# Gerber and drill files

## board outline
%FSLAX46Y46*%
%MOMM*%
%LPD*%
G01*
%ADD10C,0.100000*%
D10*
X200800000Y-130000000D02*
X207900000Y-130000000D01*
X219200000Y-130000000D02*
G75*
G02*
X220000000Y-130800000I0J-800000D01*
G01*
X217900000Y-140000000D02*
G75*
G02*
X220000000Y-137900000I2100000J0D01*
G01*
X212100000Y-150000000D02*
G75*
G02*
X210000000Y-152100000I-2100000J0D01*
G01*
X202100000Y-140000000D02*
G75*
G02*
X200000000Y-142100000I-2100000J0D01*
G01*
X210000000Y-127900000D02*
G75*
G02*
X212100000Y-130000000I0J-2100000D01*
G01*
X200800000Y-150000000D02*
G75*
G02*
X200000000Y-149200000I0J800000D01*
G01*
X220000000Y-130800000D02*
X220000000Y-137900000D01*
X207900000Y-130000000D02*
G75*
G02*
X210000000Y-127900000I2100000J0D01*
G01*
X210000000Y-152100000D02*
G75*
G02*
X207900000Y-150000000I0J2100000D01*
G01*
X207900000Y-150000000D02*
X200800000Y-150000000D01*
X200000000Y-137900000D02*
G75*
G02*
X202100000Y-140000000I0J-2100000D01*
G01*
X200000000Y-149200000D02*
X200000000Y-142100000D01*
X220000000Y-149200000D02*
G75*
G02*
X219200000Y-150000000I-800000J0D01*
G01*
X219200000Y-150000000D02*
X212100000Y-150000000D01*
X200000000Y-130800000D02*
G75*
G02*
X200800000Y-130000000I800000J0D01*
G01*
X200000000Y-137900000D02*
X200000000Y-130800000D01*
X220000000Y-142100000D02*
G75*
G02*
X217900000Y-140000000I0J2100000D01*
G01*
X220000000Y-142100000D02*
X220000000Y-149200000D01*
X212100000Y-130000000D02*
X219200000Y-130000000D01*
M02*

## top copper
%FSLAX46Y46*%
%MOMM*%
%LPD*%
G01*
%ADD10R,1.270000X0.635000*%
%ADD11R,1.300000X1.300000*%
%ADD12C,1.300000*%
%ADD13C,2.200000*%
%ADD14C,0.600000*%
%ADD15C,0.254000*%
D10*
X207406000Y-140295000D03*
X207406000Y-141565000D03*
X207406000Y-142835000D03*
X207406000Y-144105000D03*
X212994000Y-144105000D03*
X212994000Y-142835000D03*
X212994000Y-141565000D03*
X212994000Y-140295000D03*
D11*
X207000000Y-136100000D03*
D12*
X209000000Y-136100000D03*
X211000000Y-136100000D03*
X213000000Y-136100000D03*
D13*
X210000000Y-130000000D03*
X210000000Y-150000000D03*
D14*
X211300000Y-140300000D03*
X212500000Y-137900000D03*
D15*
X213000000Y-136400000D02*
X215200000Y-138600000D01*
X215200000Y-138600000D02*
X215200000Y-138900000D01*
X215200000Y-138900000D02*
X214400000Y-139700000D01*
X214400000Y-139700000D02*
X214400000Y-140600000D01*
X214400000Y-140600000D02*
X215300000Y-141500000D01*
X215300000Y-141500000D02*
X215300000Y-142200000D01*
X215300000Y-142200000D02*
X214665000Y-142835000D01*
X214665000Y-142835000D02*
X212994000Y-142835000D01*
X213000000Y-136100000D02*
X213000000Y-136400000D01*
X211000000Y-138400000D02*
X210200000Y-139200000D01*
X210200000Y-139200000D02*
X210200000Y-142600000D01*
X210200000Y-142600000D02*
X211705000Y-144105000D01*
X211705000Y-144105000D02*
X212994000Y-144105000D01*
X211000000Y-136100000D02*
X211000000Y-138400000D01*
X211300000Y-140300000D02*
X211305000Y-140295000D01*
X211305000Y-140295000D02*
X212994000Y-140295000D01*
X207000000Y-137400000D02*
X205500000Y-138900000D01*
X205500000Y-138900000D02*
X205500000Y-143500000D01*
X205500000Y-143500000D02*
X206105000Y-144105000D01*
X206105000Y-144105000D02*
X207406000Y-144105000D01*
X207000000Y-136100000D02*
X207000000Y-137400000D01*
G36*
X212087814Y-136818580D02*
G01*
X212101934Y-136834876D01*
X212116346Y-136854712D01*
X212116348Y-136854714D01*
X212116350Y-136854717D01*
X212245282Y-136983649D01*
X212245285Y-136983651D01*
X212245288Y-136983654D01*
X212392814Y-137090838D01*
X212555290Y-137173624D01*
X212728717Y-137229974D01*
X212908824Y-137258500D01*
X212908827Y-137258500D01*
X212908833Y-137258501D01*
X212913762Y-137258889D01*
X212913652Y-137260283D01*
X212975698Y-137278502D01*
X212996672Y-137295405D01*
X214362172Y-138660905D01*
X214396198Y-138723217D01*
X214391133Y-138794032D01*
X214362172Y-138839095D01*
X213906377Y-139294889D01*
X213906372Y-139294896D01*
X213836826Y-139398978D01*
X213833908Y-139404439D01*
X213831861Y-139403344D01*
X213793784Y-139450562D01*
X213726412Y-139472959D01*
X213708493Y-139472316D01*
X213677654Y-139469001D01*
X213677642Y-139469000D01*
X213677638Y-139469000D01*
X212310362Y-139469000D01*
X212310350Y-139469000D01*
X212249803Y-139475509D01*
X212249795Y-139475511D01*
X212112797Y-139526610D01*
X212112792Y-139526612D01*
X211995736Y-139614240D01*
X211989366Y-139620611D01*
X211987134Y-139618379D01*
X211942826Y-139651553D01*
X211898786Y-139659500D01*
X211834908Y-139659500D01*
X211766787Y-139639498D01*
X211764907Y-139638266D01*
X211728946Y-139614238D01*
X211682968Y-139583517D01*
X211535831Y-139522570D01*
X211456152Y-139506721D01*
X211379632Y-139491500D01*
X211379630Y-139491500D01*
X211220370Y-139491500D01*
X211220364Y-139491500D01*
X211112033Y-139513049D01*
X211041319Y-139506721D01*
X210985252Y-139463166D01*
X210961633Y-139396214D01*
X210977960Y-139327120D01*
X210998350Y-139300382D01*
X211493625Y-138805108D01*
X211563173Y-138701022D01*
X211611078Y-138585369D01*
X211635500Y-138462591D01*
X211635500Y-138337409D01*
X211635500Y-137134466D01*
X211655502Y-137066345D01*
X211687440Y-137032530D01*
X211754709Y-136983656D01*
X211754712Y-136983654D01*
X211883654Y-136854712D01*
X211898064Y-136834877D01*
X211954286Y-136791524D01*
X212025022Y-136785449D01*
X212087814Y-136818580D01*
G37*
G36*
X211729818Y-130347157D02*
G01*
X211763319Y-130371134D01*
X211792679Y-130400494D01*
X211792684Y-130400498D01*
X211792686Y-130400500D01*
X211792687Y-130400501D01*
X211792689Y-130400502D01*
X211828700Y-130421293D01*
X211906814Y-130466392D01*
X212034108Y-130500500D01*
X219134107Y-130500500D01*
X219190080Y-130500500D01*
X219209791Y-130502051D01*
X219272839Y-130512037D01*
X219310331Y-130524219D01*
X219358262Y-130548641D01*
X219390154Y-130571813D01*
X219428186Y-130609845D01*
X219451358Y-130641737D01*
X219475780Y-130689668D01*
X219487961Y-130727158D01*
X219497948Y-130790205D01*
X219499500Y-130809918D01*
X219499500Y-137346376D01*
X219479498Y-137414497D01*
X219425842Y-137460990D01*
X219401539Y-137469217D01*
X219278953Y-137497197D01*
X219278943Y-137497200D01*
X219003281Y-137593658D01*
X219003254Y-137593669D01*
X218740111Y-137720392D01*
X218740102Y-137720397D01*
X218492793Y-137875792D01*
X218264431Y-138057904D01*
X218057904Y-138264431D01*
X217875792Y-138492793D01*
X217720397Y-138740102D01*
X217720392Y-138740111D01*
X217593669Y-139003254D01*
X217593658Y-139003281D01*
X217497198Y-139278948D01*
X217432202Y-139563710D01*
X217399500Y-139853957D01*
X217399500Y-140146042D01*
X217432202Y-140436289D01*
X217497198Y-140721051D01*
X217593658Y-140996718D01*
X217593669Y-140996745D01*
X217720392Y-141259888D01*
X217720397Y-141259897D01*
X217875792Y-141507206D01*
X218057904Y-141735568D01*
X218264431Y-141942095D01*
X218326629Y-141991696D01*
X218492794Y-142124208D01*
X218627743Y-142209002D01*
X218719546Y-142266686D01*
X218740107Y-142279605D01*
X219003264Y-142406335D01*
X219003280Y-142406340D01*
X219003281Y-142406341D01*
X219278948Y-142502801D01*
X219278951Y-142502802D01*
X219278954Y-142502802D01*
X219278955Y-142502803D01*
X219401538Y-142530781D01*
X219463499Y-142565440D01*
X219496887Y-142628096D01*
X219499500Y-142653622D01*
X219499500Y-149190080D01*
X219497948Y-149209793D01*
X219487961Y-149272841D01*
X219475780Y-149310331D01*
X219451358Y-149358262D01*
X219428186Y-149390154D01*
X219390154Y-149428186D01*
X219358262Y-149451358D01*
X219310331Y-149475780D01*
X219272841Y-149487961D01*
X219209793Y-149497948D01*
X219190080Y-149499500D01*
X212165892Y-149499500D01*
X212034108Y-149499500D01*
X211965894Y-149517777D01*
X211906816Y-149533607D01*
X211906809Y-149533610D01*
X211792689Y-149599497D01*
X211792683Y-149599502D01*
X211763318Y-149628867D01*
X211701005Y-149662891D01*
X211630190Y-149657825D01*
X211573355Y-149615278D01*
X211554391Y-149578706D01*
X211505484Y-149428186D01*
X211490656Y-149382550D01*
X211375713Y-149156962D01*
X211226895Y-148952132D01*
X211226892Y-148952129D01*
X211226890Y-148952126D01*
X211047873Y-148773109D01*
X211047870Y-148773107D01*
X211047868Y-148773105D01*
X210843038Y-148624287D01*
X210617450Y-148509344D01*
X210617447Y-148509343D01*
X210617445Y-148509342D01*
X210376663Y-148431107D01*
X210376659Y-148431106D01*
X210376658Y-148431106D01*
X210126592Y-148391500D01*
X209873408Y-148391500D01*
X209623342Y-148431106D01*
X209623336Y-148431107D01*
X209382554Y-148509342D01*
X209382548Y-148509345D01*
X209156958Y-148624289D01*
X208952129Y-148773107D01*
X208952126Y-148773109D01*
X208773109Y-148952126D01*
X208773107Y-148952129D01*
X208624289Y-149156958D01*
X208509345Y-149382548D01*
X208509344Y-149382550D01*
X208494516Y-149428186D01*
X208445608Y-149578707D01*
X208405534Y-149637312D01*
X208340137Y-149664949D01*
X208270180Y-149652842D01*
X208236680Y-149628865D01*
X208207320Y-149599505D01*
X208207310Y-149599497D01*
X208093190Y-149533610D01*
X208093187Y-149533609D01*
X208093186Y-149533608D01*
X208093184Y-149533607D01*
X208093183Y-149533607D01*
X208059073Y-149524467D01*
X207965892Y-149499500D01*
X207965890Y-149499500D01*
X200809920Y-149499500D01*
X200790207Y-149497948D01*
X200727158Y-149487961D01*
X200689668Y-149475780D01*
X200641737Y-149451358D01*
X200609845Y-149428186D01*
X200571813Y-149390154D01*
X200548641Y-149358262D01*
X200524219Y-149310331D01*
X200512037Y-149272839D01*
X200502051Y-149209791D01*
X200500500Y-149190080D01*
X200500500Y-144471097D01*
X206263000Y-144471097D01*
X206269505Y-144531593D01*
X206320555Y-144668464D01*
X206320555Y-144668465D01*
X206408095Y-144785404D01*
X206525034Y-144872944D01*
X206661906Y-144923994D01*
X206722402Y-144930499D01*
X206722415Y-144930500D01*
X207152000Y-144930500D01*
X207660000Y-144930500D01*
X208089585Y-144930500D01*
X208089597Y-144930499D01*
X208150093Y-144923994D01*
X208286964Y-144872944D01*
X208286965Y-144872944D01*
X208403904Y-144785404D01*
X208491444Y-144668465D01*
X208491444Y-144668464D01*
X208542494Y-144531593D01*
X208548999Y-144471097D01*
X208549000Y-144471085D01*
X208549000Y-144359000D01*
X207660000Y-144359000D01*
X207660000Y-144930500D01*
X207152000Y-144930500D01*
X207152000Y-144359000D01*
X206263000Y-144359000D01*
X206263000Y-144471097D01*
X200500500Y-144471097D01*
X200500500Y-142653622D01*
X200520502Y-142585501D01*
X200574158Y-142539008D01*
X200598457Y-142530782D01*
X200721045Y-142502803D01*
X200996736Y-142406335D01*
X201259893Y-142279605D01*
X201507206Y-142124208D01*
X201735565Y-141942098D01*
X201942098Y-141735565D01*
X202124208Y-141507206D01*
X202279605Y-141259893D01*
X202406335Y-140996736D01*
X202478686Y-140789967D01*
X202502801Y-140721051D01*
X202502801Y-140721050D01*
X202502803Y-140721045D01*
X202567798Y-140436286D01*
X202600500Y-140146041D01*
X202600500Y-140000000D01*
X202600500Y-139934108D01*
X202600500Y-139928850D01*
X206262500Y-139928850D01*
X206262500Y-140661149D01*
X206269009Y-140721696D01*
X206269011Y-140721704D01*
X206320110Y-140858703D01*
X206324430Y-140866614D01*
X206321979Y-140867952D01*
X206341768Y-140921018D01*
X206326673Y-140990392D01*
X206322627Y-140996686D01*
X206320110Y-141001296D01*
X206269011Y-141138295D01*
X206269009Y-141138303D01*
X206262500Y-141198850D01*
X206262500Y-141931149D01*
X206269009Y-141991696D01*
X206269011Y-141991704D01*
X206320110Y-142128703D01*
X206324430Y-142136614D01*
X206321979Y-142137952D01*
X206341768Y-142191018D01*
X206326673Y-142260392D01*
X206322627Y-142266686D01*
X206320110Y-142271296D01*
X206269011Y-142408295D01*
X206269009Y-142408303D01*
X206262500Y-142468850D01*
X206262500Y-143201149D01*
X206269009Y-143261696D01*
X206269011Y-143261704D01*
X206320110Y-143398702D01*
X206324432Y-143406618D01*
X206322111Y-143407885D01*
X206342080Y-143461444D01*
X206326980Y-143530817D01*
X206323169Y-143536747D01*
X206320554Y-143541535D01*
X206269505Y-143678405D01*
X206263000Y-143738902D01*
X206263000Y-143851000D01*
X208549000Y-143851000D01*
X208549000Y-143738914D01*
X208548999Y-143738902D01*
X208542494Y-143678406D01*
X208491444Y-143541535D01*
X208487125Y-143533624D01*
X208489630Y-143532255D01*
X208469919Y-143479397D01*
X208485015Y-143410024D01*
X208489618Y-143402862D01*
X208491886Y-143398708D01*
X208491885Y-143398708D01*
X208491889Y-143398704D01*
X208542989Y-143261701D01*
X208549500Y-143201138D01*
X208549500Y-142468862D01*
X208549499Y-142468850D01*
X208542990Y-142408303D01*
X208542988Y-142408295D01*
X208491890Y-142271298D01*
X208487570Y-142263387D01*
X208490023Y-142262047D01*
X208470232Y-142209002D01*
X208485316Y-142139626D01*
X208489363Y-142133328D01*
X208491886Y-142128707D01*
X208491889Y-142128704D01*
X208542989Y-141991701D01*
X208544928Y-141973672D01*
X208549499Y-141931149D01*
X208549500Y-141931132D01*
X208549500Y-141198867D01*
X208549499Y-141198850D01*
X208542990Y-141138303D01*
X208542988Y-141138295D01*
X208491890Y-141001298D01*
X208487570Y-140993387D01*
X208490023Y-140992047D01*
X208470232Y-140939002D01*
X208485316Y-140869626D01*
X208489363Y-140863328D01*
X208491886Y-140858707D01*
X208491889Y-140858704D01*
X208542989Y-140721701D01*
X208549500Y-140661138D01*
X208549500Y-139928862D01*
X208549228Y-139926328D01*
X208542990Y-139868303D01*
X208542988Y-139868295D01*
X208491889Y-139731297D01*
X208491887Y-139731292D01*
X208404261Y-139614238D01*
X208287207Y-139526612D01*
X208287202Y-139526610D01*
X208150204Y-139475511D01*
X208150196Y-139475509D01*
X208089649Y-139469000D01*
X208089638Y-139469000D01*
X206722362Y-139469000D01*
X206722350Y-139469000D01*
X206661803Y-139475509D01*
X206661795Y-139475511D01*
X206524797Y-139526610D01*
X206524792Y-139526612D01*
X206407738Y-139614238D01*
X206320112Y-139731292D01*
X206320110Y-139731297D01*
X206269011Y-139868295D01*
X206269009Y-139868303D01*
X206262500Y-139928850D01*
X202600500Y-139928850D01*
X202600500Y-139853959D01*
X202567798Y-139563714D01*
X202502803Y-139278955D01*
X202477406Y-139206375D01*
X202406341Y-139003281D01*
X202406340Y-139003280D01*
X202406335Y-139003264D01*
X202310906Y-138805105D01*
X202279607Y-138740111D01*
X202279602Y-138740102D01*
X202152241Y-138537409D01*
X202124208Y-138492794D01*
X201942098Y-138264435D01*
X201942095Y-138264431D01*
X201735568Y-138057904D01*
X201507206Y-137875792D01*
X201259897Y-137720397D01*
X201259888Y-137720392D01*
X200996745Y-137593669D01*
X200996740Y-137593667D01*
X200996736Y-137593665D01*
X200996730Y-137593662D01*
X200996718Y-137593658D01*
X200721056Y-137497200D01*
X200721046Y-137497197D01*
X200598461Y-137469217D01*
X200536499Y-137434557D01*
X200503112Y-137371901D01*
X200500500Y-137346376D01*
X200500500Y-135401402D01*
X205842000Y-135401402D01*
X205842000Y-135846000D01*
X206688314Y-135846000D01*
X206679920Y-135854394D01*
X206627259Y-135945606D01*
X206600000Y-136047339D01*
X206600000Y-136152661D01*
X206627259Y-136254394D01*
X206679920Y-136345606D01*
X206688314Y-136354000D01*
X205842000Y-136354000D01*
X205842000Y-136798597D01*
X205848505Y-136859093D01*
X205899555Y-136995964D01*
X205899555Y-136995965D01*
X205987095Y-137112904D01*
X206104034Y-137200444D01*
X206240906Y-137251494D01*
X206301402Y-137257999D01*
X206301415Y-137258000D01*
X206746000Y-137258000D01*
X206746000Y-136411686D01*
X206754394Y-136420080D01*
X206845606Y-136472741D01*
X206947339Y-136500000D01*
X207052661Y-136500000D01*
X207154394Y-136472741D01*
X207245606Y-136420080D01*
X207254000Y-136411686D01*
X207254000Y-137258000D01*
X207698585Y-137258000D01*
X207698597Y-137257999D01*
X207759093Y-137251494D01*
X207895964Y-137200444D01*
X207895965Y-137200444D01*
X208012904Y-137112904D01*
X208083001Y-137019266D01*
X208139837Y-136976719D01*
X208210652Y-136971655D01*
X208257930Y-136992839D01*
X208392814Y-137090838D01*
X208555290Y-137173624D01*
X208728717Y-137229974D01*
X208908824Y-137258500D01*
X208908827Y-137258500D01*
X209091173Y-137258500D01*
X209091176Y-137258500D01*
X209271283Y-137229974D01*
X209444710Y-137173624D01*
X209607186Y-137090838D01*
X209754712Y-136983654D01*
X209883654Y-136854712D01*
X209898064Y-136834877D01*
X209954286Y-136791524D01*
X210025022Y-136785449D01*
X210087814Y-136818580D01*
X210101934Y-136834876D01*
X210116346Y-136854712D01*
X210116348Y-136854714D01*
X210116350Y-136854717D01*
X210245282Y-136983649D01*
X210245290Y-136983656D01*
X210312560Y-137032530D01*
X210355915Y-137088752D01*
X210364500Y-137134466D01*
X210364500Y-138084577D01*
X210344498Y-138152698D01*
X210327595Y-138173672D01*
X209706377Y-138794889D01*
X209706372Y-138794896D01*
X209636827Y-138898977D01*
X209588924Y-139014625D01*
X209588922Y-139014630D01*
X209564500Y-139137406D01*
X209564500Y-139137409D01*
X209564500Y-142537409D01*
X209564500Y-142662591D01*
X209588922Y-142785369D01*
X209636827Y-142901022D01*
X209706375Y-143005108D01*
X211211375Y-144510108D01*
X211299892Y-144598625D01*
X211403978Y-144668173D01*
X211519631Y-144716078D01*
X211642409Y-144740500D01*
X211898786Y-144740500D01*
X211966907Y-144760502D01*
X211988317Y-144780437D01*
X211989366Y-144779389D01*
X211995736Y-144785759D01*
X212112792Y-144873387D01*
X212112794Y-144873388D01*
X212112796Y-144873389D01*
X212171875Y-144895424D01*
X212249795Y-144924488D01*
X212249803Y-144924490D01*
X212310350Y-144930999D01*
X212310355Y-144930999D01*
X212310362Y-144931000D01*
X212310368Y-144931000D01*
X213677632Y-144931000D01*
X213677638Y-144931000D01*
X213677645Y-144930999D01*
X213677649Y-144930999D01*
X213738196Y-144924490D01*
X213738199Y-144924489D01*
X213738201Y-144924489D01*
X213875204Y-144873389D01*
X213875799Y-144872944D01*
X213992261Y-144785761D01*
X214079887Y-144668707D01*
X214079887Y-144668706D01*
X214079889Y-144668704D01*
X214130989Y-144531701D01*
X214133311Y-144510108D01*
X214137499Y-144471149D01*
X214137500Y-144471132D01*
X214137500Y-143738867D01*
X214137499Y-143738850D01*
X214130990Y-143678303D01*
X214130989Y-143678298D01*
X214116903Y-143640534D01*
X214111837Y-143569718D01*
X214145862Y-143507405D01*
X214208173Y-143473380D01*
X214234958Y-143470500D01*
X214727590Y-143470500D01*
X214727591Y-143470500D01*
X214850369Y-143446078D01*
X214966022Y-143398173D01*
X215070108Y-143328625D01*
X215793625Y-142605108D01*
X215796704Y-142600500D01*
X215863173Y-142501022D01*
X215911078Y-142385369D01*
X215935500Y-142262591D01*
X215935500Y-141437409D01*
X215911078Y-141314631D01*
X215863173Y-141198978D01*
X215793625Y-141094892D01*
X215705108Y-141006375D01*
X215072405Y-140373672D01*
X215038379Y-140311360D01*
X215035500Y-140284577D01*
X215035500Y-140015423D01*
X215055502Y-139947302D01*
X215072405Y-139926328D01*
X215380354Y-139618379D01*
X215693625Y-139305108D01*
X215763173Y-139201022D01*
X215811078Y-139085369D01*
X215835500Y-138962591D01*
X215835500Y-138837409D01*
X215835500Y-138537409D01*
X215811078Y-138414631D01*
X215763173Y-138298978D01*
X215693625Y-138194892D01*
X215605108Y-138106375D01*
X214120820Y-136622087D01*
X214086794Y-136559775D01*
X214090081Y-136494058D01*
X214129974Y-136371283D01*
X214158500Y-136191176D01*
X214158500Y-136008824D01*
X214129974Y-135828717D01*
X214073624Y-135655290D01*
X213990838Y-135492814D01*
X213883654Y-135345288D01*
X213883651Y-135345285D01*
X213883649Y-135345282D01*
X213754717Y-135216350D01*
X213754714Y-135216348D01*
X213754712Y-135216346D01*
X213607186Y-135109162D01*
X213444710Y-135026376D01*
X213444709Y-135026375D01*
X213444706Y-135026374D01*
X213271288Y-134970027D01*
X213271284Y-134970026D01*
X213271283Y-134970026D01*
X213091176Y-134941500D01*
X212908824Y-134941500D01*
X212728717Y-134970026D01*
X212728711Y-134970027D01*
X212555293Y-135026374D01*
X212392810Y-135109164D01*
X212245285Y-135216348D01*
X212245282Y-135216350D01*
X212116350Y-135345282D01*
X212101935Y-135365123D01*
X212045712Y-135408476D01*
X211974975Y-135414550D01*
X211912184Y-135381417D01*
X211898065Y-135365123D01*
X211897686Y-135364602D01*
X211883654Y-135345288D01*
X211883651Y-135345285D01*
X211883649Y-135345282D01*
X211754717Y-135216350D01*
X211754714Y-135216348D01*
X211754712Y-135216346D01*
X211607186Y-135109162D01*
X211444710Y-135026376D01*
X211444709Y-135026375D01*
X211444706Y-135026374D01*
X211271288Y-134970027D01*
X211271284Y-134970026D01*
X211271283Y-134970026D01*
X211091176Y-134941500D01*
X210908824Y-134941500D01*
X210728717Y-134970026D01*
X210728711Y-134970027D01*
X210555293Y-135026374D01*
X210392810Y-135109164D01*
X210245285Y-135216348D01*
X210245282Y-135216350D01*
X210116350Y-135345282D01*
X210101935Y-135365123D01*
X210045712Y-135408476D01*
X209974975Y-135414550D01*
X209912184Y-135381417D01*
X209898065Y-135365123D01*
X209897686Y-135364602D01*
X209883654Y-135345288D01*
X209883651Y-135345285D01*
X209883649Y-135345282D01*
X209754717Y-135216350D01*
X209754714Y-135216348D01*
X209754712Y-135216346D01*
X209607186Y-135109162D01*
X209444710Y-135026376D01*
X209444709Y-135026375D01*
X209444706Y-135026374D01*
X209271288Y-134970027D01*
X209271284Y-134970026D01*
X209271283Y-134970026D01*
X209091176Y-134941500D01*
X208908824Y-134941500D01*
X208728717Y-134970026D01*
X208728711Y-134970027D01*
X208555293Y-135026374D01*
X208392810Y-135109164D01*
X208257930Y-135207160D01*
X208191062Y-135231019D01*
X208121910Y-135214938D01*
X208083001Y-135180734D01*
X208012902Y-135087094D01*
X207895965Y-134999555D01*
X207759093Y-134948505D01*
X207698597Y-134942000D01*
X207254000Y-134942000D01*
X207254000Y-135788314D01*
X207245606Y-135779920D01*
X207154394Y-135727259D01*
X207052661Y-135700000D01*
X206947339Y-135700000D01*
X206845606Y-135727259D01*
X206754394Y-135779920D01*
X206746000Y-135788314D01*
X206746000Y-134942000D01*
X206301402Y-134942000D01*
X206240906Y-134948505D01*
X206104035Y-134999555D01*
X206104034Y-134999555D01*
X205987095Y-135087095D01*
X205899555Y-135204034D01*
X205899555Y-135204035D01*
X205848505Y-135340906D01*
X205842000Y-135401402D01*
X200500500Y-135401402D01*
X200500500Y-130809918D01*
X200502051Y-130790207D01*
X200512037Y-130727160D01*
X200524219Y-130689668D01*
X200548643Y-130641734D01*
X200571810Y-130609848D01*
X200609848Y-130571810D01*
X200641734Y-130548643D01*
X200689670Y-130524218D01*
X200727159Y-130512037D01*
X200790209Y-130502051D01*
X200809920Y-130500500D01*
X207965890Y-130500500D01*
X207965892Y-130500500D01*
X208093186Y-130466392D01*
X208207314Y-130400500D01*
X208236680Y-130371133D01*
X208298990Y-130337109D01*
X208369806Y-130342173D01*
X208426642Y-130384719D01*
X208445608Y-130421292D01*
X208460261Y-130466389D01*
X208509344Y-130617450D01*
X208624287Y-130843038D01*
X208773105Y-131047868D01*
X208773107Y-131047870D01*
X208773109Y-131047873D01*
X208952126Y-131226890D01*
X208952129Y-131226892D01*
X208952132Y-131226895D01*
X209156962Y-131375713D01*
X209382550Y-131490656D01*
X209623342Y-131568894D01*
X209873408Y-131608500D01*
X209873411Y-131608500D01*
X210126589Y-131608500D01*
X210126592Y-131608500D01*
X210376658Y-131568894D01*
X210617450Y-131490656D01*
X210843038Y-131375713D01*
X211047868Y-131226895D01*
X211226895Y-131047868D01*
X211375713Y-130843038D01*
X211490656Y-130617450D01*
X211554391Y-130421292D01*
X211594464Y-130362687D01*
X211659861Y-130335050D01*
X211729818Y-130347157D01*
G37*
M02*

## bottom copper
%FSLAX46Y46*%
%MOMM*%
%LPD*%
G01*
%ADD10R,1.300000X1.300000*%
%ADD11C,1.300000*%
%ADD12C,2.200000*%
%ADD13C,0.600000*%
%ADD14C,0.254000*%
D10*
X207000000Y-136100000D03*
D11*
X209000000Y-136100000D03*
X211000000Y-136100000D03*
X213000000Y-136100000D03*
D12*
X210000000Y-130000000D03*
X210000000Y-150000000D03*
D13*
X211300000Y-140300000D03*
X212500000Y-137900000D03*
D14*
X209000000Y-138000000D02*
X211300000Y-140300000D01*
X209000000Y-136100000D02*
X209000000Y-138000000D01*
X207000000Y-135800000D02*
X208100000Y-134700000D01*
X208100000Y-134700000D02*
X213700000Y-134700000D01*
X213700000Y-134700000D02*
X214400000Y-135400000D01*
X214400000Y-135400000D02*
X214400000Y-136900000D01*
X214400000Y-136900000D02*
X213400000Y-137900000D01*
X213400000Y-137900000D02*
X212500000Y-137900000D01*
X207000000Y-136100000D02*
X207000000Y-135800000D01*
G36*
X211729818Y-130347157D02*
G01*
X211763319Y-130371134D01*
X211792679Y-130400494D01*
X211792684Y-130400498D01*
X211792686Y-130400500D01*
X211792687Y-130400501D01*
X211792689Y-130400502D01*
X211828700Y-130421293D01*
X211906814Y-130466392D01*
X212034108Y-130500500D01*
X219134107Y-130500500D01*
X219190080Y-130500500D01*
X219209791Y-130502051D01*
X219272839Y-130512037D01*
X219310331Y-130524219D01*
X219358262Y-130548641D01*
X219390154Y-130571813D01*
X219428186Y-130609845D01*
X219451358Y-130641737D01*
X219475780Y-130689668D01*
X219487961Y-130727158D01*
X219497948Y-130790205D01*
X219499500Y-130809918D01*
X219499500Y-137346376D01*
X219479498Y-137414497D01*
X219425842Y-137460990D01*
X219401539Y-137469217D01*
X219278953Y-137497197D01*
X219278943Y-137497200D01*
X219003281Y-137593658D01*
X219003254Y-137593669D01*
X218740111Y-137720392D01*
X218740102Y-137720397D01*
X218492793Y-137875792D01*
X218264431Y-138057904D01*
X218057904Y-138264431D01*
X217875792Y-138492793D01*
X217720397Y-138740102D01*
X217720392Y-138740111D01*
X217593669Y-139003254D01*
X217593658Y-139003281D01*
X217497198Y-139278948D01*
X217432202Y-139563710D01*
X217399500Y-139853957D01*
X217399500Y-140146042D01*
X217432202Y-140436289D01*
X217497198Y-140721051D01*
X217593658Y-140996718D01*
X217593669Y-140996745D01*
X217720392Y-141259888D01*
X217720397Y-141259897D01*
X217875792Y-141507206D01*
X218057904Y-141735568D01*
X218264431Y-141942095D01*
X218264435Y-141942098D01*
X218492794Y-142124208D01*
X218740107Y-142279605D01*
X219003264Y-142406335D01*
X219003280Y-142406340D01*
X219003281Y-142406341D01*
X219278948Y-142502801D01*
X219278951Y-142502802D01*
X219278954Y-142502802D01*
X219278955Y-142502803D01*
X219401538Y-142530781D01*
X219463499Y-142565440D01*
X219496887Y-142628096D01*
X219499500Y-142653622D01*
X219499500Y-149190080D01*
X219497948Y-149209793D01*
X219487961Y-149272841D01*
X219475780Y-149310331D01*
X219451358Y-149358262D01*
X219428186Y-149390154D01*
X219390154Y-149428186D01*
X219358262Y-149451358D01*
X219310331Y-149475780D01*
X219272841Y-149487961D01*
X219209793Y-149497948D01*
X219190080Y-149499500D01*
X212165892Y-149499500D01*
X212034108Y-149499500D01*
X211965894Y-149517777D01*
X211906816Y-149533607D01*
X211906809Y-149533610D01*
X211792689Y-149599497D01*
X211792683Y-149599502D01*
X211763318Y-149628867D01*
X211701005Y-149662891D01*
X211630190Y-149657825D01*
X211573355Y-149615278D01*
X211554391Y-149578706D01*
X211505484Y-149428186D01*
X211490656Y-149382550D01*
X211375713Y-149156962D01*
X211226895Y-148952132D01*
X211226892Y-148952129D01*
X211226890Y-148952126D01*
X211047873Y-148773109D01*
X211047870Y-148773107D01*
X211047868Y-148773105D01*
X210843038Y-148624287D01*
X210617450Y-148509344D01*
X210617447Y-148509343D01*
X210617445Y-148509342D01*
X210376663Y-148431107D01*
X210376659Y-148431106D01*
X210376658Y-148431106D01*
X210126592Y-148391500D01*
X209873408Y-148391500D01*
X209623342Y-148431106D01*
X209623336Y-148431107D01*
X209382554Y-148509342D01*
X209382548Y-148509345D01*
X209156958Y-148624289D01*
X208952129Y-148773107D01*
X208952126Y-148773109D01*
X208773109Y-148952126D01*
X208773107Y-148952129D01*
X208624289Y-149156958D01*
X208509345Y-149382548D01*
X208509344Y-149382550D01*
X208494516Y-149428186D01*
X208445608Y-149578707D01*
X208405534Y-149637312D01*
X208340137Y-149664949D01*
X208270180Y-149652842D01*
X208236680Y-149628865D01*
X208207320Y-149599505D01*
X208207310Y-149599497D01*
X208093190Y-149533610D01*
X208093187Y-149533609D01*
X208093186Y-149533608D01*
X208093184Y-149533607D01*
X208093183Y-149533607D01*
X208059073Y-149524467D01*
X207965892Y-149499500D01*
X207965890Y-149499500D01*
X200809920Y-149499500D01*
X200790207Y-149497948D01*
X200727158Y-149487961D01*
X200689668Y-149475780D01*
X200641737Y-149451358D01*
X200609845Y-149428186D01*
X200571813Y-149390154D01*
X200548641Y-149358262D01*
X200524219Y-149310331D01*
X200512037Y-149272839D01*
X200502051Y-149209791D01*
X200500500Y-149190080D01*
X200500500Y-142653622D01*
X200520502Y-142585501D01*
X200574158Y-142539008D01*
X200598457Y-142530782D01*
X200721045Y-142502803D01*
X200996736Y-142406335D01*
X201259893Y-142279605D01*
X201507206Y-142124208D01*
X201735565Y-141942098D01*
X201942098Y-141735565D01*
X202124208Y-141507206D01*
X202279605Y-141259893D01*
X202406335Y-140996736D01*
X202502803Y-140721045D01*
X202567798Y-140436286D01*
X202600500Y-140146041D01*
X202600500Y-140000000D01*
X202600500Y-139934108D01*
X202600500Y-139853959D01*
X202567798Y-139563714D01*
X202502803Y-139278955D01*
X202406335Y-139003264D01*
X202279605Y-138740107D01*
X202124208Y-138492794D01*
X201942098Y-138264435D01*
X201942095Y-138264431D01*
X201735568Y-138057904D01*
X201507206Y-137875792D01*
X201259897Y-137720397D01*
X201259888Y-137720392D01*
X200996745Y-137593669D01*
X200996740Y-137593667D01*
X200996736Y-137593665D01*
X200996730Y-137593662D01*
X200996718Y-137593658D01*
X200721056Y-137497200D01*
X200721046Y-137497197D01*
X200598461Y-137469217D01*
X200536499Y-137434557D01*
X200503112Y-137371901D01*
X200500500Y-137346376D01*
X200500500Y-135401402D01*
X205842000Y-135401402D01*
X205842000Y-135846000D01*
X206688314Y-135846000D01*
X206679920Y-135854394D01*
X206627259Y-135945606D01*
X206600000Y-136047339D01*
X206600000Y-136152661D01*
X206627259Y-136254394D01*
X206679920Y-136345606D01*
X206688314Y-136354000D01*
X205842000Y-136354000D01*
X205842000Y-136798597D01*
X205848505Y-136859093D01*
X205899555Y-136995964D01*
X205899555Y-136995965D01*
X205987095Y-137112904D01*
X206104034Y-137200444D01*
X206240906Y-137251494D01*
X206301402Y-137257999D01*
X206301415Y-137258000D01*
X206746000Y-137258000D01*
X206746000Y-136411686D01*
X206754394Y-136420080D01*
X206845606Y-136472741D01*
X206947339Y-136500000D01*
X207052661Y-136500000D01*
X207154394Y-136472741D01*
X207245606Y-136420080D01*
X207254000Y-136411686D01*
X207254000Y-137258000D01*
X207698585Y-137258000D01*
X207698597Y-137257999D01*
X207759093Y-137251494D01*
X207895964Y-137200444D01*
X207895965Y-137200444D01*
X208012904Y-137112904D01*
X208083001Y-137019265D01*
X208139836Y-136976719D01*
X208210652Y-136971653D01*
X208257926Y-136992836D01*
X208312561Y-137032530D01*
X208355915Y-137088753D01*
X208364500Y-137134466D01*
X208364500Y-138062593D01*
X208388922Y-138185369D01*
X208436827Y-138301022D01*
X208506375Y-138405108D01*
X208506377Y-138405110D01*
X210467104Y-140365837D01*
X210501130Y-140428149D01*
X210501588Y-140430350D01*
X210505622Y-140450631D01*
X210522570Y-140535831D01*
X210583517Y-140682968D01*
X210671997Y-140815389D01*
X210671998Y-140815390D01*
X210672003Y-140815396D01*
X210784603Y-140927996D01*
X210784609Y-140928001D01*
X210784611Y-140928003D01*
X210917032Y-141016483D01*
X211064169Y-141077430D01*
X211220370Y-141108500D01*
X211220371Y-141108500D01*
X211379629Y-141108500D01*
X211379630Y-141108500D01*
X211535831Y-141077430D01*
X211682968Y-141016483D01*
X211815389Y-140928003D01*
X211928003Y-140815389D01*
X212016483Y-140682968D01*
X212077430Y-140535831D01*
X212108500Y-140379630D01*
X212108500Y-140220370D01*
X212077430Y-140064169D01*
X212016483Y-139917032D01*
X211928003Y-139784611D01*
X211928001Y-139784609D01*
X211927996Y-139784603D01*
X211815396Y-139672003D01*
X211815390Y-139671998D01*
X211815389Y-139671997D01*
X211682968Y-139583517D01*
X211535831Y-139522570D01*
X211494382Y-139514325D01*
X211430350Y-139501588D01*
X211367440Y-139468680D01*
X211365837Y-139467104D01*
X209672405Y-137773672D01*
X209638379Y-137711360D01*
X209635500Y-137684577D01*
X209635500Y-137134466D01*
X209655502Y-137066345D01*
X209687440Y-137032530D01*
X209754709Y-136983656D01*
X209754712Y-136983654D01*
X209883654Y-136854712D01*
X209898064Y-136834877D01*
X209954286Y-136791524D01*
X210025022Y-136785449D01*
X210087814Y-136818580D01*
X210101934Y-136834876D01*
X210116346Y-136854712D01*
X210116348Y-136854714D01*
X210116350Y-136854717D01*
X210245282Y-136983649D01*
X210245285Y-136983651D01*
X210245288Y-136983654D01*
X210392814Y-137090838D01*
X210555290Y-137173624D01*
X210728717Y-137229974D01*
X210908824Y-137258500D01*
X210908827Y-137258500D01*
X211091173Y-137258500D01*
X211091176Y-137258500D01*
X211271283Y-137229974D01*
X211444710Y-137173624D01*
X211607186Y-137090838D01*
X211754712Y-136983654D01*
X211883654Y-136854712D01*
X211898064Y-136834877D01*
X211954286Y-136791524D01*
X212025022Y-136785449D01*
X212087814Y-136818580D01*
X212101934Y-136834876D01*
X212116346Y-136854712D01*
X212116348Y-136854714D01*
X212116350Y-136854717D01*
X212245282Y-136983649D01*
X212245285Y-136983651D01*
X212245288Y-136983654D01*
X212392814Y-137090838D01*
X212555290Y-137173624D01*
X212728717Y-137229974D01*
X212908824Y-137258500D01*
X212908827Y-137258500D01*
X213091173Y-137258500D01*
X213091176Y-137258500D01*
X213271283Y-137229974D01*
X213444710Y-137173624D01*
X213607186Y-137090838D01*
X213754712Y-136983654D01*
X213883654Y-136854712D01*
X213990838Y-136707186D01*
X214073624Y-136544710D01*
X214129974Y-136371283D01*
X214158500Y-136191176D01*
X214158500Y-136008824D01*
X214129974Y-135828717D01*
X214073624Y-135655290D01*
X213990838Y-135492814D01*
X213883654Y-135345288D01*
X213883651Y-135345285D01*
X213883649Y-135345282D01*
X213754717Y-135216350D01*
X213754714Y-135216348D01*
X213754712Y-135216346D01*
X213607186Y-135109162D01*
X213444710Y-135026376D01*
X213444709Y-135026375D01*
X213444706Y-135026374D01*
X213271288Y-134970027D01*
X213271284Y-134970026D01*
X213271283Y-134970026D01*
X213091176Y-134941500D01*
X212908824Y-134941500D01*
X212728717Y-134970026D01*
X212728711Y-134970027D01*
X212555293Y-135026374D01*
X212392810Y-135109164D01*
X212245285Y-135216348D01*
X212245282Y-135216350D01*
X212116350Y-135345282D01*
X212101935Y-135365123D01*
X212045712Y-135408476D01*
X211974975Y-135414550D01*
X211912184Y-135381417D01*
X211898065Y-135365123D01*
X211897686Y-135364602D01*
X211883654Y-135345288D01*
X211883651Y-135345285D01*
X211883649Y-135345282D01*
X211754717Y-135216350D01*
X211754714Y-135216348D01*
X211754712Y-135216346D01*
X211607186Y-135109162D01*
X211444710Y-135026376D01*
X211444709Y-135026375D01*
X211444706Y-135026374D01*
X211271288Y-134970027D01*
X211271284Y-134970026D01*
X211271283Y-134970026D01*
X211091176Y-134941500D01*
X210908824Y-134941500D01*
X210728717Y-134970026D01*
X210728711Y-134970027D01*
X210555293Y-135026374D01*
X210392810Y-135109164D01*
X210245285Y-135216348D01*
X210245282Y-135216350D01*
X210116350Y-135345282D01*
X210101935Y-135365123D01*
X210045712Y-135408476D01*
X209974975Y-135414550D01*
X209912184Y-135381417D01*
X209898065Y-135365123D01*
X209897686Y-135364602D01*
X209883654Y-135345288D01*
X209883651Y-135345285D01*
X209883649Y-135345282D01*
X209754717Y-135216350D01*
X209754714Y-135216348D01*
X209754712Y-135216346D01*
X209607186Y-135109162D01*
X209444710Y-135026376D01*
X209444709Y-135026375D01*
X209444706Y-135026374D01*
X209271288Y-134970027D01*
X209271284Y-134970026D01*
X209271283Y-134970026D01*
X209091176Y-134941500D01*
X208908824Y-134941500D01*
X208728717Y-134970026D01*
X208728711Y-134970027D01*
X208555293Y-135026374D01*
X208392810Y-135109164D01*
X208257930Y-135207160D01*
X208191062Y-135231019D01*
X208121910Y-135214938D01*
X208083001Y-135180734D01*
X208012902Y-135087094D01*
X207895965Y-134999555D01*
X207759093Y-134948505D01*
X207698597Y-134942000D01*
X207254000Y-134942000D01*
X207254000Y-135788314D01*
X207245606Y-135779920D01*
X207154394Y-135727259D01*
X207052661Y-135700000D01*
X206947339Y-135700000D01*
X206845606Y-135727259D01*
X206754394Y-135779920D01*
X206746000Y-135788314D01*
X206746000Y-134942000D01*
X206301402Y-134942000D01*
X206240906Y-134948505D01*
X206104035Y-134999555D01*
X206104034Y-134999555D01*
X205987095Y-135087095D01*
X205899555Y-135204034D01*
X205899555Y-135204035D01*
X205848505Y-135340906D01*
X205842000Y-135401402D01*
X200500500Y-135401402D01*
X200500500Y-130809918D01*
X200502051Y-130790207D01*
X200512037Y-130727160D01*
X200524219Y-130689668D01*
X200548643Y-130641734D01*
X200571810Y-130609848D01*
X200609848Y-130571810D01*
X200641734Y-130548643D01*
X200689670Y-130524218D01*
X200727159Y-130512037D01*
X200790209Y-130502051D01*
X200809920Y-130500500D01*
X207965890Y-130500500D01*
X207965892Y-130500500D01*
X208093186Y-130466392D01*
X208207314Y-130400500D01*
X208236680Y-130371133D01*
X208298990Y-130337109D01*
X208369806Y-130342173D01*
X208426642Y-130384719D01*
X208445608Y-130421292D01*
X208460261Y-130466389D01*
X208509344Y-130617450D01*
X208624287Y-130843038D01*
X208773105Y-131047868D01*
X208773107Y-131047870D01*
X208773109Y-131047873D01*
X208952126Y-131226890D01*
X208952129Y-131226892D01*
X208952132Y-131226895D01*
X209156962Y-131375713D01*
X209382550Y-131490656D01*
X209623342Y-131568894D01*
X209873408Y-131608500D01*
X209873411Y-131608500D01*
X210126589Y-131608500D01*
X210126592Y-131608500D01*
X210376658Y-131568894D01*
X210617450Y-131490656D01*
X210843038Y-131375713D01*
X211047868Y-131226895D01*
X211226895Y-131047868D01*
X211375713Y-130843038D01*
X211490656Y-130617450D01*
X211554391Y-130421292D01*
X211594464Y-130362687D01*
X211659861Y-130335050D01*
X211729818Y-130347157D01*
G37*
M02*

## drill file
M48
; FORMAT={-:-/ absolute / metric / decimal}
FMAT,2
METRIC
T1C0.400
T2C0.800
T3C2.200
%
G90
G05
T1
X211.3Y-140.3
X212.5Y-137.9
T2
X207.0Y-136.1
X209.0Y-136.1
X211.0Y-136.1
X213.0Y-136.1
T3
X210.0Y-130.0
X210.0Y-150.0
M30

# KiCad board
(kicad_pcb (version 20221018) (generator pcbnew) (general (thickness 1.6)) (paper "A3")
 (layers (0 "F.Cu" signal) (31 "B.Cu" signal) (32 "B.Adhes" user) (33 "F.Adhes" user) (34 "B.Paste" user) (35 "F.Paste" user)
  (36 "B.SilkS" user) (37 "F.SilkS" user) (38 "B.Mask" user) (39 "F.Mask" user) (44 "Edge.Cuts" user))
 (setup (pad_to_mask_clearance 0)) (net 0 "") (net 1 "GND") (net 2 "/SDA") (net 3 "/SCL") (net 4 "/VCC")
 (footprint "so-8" (layer "F.Cu") (at 210.2 142.2 -90)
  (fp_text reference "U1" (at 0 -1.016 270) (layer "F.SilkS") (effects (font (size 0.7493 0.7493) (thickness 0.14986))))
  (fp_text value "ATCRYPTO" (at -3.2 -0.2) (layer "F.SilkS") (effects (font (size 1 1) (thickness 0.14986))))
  (pad "1" smd rect (at -1.905 2.794 270) (size 0.635 1.27) (layers "F.Cu" "F.Paste" "F.Mask"))
  (pad "2" smd rect (at -0.635 2.794 270) (size 0.635 1.27) (layers "F.Cu" "F.Paste" "F.Mask"))
  (pad "3" smd rect (at 0.635 2.794 270) (size 0.635 1.27) (layers "F.Cu" "F.Paste" "F.Mask"))
  (pad "4" smd rect (at 1.905 2.794 270) (size 0.635 1.27) (layers "F.Cu" "F.Paste" "F.Mask") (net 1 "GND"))
  (pad "5" smd rect (at 1.905 -2.794 270) (size 0.635 1.27) (layers "F.Cu" "F.Paste" "F.Mask") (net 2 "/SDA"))
  (pad "6" smd rect (at 0.635 -2.794 270) (size 0.635 1.27) (layers "F.Cu" "F.Paste" "F.Mask") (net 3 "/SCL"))
  (pad "7" smd rect (at -0.635 -2.794 270) (size 0.635 1.27) (layers "F.Cu" "F.Paste" "F.Mask"))
  (pad "8" smd rect (at -1.905 -2.794 270) (size 0.635 1.27) (layers "F.Cu" "F.Paste" "F.Mask") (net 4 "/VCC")))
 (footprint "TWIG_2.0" (layer "F.Cu") (at 210 136.1)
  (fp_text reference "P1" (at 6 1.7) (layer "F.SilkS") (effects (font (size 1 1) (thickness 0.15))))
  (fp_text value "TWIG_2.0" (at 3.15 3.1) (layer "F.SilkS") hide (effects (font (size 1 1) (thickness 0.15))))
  (pad "1" thru_hole rect (at -3 0) (size 1.3 1.3) (drill 0.8) (layers "*.Cu" "*.Mask" "F.SilkS") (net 1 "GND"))
  (pad "2" thru_hole circle (at -1 0) (size 1.3 1.3) (drill 0.8) (layers "*.Cu" "*.Mask" "F.SilkS") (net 4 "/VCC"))
  (pad "3" thru_hole circle (at 1 0) (size 1.3 1.3) (drill 0.8) (layers "*.Cu" "*.Mask" "F.SilkS") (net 2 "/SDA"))
  (pad "4" thru_hole circle (at 3 0) (size 1.3 1.3) (drill 0.8) (layers "*.Cu" "*.Mask" "F.SilkS") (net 3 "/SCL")))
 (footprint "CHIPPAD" (layer "F.Cu") (at 202.9 147.5)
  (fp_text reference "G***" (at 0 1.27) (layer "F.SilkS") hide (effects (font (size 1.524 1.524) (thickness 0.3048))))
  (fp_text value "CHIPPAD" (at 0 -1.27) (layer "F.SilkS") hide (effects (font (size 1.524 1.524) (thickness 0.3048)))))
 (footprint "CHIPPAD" (layer "F.Cu") (at 209.1 147.5)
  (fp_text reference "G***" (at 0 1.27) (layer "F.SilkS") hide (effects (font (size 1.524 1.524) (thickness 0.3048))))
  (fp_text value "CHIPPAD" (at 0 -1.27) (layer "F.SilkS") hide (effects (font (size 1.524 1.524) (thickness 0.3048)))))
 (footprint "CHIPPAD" (layer "F.Cu") (at 215 147.5)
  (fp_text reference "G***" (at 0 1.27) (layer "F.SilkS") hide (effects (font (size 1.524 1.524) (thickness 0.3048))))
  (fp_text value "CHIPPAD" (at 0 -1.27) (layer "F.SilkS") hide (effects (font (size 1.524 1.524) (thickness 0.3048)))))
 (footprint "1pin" (layer "F.Cu") (at 210 130)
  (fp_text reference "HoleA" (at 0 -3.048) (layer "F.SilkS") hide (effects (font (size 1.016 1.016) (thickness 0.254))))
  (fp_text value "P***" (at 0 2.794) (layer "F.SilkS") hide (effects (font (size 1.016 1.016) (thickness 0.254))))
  (pad "1" thru_hole circle (at 0 0) (size 2.2 2.2) (drill 2.2) (layers "*.Cu" "*.Mask" "F.SilkS")))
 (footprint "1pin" (layer "F.Cu") (at 210 150)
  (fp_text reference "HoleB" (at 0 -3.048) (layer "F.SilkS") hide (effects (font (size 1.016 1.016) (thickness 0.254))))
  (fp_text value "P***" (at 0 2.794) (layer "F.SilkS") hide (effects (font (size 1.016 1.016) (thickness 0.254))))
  (pad "1" thru_hole circle (at 0 0) (size 2.2 2.2) (drill 2.2) (layers "*.Cu" "*.Mask" "F.SilkS")))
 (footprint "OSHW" (layer "B.Cu") (at 216.3 133.2)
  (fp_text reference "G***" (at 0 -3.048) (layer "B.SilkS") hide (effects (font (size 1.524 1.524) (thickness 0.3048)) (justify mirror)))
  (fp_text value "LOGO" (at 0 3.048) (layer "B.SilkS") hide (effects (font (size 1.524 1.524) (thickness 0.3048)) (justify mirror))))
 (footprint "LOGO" (layer "B.Cu") (at 215.9 146.7)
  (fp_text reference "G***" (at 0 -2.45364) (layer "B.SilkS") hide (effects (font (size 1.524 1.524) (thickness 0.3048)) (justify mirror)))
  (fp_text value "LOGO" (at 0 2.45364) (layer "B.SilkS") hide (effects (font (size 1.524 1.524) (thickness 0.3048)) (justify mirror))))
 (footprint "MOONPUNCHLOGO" (layer "B.Cu") (at 211.4 141.4)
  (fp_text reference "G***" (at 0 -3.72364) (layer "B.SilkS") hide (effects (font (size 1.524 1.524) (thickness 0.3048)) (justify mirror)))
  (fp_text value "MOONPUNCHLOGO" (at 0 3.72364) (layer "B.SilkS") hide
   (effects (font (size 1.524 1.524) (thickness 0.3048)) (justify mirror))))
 (gr_line (start 200.8 130) (end 207.9 130) (stroke (width 0.1) (type solid)) (layer "Edge.Cuts"))
 (gr_arc (start 219.2 130) (mid 219.765685 130.234315) (end 220 130.8) (stroke (width 0.1) (type solid)) (layer "Edge.Cuts"))
 (gr_arc (start 217.9 140) (mid 218.515076 138.515076) (end 220 137.9) (stroke (width 0.1) (type solid)) (layer "Edge.Cuts"))
 (gr_arc (start 212.1 150) (mid 211.484924 151.484924) (end 210 152.1) (stroke (width 0.1) (type solid)) (layer "Edge.Cuts"))
 (gr_arc (start 202.1 140) (mid 201.484924 141.484924) (end 200 142.1) (stroke (width 0.1) (type solid)) (layer "Edge.Cuts"))
 (gr_arc (start 210 127.9) (mid 211.484924 128.515076) (end 212.1 130) (stroke (width 0.1) (type solid)) (layer "Edge.Cuts"))
 (gr_arc (start 200.8 150) (mid 200.234315 149.765685) (end 200 149.2) (stroke (width 0.1) (type solid)) (layer "Edge.Cuts"))
 (gr_line (start 220 130.8) (end 220 137.9) (stroke (width 0.1) (type solid)) (layer "Edge.Cuts"))
 (gr_arc (start 207.9 130) (mid 208.515076 128.515076) (end 210 127.9) (stroke (width 0.1) (type solid)) (layer "Edge.Cuts"))
 (gr_arc (start 210 152.1) (mid 208.515076 151.484924) (end 207.9 150) (stroke (width 0.1) (type solid)) (layer "Edge.Cuts"))
 (gr_line (start 207.9 150) (end 200.8 150) (stroke (width 0.1) (type solid)) (layer "Edge.Cuts"))
 (gr_arc (start 200 137.9) (mid 201.484924 138.515076) (end 202.1 140) (stroke (width 0.1) (type solid)) (layer "Edge.Cuts"))
 (gr_line (start 200 149.2) (end 200 142.1) (stroke (width 0.1) (type solid)) (layer "Edge.Cuts"))
 (gr_arc (start 220 149.2) (mid 219.765685 149.765685) (end 219.2 150) (stroke (width 0.1) (type solid)) (layer "Edge.Cuts"))
 (gr_line (start 219.2 150) (end 212.1 150) (stroke (width 0.1) (type solid)) (layer "Edge.Cuts"))
 (gr_arc (start 200 130.8) (mid 200.234315 130.234315) (end 200.8 130) (stroke (width 0.1) (type solid)) (layer "Edge.Cuts"))
 (gr_line (start 200 137.9) (end 200 130.8) (stroke (width 0.1) (type solid)) (layer "Edge.Cuts"))
 (gr_arc (start 220 142.1) (mid 218.515076 141.484924) (end 217.9 140) (stroke (width 0.1) (type solid)) (layer "Edge.Cuts"))
 (gr_line (start 220 142.1) (end 220 149.2) (stroke (width 0.1) (type solid)) (layer "Edge.Cuts"))
 (gr_line (start 212.1 130) (end 219.2 130) (stroke (width 0.1) (type solid)) (layer "Edge.Cuts"))
 (segment (start 213 136.4) (end 215.2 138.6) (width 0.254) (layer "F.Cu") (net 3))
 (segment (start 215.2 138.6) (end 215.2 138.9) (width 0.254) (layer "F.Cu") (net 3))
 (segment (start 215.2 138.9) (end 214.4 139.7) (width 0.254) (layer "F.Cu") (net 3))
 (segment (start 214.4 139.7) (end 214.4 140.6) (width 0.254) (layer "F.Cu") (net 3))
 (segment (start 214.4 140.6) (end 215.3 141.5) (width 0.254) (layer "F.Cu") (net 3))
 (segment (start 215.3 141.5) (end 215.3 142.2) (width 0.254) (layer "F.Cu") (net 3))
 (segment (start 215.3 142.2) (end 214.665 142.835) (width 0.254) (layer "F.Cu") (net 3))
 (segment (start 214.665 142.835) (end 212.994 142.835) (width 0.254) (layer "F.Cu") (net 3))
 (segment (start 213 136.1) (end 213 136.4) (width 0.254) (layer "F.Cu") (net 3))
 (segment (start 211 138.4) (end 210.2 139.2) (width 0.254) (layer "F.Cu") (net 2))
 (segment (start 210.2 139.2) (end 210.2 142.6) (width 0.254) (layer "F.Cu") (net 2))
 (segment (start 210.2 142.6) (end 211.705 144.105) (width 0.254) (layer "F.Cu") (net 2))
 (segment (start 211.705 144.105) (end 212.994 144.105) (width 0.254) (layer "F.Cu") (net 2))
 (segment (start 211 136.1) (end 211 138.4) (width 0.254) (layer "F.Cu") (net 2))
 (segment (start 211.3 140.3) (end 211.305 140.295) (width 0.254) (layer "F.Cu") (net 4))
 (segment (start 211.305 140.295) (end 212.994 140.295) (width 0.254) (layer "F.Cu") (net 4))
 (via (at 211.3 140.3) (size 0.6) (drill 0.4) (layers "F.Cu" "B.Cu") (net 4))
 (segment (start 209 138) (end 211.3 140.3) (width 0.254) (layer "B.Cu") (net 4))
 (segment (start 209 136.1) (end 209 138) (width 0.254) (layer "B.Cu") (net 4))
 (segment (start 207 137.4) (end 205.5 138.9) (width 0.254) (layer "F.Cu") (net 1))
 (segment (start 205.5 138.9) (end 205.5 143.5) (width 0.254) (layer "F.Cu") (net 1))
 (segment (start 205.5 143.5) (end 206.105 144.105) (width 0.254) (layer "F.Cu") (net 1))
 (segment (start 206.105 144.105) (end 207.406 144.105) (width 0.254) (layer "F.Cu") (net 1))
 (segment (start 207 136.1) (end 207 137.4) (width 0.254) (layer "F.Cu") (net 1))
 (via (at 212.5 137.9) (size 0.6) (drill 0.4) (layers "F.Cu" "B.Cu") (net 1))
 (segment (start 207 135.8) (end 208.1 134.7) (width 0.254) (layer "B.Cu") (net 1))
 (segment (start 208.1 134.7) (end 213.7 134.7) (width 0.254) (layer "B.Cu") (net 1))
 (segment (start 213.7 134.7) (end 214.4 135.4) (width 0.254) (layer "B.Cu") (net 1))
 (segment (start 214.4 135.4) (end 214.4 136.9) (width 0.254) (layer "B.Cu") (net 1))
 (segment (start 214.4 136.9) (end 213.4 137.9) (width 0.254) (layer "B.Cu") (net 1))
 (segment (start 213.4 137.9) (end 212.5 137.9) (width 0.254) (layer "B.Cu") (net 1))
 (segment (start 207 136.1) (end 207 135.8) (width 0.254) (layer "B.Cu") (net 1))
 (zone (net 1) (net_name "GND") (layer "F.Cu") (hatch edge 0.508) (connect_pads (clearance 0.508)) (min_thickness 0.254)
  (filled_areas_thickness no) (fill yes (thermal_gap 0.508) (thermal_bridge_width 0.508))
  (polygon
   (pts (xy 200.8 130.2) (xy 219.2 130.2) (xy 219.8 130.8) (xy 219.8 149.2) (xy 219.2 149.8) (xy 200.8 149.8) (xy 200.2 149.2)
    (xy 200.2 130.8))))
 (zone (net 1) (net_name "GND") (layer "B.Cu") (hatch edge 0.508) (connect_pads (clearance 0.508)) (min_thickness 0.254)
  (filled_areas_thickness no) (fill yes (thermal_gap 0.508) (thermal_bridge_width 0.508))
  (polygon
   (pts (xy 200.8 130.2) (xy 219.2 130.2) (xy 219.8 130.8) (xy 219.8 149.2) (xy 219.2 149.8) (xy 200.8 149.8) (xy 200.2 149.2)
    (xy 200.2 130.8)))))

